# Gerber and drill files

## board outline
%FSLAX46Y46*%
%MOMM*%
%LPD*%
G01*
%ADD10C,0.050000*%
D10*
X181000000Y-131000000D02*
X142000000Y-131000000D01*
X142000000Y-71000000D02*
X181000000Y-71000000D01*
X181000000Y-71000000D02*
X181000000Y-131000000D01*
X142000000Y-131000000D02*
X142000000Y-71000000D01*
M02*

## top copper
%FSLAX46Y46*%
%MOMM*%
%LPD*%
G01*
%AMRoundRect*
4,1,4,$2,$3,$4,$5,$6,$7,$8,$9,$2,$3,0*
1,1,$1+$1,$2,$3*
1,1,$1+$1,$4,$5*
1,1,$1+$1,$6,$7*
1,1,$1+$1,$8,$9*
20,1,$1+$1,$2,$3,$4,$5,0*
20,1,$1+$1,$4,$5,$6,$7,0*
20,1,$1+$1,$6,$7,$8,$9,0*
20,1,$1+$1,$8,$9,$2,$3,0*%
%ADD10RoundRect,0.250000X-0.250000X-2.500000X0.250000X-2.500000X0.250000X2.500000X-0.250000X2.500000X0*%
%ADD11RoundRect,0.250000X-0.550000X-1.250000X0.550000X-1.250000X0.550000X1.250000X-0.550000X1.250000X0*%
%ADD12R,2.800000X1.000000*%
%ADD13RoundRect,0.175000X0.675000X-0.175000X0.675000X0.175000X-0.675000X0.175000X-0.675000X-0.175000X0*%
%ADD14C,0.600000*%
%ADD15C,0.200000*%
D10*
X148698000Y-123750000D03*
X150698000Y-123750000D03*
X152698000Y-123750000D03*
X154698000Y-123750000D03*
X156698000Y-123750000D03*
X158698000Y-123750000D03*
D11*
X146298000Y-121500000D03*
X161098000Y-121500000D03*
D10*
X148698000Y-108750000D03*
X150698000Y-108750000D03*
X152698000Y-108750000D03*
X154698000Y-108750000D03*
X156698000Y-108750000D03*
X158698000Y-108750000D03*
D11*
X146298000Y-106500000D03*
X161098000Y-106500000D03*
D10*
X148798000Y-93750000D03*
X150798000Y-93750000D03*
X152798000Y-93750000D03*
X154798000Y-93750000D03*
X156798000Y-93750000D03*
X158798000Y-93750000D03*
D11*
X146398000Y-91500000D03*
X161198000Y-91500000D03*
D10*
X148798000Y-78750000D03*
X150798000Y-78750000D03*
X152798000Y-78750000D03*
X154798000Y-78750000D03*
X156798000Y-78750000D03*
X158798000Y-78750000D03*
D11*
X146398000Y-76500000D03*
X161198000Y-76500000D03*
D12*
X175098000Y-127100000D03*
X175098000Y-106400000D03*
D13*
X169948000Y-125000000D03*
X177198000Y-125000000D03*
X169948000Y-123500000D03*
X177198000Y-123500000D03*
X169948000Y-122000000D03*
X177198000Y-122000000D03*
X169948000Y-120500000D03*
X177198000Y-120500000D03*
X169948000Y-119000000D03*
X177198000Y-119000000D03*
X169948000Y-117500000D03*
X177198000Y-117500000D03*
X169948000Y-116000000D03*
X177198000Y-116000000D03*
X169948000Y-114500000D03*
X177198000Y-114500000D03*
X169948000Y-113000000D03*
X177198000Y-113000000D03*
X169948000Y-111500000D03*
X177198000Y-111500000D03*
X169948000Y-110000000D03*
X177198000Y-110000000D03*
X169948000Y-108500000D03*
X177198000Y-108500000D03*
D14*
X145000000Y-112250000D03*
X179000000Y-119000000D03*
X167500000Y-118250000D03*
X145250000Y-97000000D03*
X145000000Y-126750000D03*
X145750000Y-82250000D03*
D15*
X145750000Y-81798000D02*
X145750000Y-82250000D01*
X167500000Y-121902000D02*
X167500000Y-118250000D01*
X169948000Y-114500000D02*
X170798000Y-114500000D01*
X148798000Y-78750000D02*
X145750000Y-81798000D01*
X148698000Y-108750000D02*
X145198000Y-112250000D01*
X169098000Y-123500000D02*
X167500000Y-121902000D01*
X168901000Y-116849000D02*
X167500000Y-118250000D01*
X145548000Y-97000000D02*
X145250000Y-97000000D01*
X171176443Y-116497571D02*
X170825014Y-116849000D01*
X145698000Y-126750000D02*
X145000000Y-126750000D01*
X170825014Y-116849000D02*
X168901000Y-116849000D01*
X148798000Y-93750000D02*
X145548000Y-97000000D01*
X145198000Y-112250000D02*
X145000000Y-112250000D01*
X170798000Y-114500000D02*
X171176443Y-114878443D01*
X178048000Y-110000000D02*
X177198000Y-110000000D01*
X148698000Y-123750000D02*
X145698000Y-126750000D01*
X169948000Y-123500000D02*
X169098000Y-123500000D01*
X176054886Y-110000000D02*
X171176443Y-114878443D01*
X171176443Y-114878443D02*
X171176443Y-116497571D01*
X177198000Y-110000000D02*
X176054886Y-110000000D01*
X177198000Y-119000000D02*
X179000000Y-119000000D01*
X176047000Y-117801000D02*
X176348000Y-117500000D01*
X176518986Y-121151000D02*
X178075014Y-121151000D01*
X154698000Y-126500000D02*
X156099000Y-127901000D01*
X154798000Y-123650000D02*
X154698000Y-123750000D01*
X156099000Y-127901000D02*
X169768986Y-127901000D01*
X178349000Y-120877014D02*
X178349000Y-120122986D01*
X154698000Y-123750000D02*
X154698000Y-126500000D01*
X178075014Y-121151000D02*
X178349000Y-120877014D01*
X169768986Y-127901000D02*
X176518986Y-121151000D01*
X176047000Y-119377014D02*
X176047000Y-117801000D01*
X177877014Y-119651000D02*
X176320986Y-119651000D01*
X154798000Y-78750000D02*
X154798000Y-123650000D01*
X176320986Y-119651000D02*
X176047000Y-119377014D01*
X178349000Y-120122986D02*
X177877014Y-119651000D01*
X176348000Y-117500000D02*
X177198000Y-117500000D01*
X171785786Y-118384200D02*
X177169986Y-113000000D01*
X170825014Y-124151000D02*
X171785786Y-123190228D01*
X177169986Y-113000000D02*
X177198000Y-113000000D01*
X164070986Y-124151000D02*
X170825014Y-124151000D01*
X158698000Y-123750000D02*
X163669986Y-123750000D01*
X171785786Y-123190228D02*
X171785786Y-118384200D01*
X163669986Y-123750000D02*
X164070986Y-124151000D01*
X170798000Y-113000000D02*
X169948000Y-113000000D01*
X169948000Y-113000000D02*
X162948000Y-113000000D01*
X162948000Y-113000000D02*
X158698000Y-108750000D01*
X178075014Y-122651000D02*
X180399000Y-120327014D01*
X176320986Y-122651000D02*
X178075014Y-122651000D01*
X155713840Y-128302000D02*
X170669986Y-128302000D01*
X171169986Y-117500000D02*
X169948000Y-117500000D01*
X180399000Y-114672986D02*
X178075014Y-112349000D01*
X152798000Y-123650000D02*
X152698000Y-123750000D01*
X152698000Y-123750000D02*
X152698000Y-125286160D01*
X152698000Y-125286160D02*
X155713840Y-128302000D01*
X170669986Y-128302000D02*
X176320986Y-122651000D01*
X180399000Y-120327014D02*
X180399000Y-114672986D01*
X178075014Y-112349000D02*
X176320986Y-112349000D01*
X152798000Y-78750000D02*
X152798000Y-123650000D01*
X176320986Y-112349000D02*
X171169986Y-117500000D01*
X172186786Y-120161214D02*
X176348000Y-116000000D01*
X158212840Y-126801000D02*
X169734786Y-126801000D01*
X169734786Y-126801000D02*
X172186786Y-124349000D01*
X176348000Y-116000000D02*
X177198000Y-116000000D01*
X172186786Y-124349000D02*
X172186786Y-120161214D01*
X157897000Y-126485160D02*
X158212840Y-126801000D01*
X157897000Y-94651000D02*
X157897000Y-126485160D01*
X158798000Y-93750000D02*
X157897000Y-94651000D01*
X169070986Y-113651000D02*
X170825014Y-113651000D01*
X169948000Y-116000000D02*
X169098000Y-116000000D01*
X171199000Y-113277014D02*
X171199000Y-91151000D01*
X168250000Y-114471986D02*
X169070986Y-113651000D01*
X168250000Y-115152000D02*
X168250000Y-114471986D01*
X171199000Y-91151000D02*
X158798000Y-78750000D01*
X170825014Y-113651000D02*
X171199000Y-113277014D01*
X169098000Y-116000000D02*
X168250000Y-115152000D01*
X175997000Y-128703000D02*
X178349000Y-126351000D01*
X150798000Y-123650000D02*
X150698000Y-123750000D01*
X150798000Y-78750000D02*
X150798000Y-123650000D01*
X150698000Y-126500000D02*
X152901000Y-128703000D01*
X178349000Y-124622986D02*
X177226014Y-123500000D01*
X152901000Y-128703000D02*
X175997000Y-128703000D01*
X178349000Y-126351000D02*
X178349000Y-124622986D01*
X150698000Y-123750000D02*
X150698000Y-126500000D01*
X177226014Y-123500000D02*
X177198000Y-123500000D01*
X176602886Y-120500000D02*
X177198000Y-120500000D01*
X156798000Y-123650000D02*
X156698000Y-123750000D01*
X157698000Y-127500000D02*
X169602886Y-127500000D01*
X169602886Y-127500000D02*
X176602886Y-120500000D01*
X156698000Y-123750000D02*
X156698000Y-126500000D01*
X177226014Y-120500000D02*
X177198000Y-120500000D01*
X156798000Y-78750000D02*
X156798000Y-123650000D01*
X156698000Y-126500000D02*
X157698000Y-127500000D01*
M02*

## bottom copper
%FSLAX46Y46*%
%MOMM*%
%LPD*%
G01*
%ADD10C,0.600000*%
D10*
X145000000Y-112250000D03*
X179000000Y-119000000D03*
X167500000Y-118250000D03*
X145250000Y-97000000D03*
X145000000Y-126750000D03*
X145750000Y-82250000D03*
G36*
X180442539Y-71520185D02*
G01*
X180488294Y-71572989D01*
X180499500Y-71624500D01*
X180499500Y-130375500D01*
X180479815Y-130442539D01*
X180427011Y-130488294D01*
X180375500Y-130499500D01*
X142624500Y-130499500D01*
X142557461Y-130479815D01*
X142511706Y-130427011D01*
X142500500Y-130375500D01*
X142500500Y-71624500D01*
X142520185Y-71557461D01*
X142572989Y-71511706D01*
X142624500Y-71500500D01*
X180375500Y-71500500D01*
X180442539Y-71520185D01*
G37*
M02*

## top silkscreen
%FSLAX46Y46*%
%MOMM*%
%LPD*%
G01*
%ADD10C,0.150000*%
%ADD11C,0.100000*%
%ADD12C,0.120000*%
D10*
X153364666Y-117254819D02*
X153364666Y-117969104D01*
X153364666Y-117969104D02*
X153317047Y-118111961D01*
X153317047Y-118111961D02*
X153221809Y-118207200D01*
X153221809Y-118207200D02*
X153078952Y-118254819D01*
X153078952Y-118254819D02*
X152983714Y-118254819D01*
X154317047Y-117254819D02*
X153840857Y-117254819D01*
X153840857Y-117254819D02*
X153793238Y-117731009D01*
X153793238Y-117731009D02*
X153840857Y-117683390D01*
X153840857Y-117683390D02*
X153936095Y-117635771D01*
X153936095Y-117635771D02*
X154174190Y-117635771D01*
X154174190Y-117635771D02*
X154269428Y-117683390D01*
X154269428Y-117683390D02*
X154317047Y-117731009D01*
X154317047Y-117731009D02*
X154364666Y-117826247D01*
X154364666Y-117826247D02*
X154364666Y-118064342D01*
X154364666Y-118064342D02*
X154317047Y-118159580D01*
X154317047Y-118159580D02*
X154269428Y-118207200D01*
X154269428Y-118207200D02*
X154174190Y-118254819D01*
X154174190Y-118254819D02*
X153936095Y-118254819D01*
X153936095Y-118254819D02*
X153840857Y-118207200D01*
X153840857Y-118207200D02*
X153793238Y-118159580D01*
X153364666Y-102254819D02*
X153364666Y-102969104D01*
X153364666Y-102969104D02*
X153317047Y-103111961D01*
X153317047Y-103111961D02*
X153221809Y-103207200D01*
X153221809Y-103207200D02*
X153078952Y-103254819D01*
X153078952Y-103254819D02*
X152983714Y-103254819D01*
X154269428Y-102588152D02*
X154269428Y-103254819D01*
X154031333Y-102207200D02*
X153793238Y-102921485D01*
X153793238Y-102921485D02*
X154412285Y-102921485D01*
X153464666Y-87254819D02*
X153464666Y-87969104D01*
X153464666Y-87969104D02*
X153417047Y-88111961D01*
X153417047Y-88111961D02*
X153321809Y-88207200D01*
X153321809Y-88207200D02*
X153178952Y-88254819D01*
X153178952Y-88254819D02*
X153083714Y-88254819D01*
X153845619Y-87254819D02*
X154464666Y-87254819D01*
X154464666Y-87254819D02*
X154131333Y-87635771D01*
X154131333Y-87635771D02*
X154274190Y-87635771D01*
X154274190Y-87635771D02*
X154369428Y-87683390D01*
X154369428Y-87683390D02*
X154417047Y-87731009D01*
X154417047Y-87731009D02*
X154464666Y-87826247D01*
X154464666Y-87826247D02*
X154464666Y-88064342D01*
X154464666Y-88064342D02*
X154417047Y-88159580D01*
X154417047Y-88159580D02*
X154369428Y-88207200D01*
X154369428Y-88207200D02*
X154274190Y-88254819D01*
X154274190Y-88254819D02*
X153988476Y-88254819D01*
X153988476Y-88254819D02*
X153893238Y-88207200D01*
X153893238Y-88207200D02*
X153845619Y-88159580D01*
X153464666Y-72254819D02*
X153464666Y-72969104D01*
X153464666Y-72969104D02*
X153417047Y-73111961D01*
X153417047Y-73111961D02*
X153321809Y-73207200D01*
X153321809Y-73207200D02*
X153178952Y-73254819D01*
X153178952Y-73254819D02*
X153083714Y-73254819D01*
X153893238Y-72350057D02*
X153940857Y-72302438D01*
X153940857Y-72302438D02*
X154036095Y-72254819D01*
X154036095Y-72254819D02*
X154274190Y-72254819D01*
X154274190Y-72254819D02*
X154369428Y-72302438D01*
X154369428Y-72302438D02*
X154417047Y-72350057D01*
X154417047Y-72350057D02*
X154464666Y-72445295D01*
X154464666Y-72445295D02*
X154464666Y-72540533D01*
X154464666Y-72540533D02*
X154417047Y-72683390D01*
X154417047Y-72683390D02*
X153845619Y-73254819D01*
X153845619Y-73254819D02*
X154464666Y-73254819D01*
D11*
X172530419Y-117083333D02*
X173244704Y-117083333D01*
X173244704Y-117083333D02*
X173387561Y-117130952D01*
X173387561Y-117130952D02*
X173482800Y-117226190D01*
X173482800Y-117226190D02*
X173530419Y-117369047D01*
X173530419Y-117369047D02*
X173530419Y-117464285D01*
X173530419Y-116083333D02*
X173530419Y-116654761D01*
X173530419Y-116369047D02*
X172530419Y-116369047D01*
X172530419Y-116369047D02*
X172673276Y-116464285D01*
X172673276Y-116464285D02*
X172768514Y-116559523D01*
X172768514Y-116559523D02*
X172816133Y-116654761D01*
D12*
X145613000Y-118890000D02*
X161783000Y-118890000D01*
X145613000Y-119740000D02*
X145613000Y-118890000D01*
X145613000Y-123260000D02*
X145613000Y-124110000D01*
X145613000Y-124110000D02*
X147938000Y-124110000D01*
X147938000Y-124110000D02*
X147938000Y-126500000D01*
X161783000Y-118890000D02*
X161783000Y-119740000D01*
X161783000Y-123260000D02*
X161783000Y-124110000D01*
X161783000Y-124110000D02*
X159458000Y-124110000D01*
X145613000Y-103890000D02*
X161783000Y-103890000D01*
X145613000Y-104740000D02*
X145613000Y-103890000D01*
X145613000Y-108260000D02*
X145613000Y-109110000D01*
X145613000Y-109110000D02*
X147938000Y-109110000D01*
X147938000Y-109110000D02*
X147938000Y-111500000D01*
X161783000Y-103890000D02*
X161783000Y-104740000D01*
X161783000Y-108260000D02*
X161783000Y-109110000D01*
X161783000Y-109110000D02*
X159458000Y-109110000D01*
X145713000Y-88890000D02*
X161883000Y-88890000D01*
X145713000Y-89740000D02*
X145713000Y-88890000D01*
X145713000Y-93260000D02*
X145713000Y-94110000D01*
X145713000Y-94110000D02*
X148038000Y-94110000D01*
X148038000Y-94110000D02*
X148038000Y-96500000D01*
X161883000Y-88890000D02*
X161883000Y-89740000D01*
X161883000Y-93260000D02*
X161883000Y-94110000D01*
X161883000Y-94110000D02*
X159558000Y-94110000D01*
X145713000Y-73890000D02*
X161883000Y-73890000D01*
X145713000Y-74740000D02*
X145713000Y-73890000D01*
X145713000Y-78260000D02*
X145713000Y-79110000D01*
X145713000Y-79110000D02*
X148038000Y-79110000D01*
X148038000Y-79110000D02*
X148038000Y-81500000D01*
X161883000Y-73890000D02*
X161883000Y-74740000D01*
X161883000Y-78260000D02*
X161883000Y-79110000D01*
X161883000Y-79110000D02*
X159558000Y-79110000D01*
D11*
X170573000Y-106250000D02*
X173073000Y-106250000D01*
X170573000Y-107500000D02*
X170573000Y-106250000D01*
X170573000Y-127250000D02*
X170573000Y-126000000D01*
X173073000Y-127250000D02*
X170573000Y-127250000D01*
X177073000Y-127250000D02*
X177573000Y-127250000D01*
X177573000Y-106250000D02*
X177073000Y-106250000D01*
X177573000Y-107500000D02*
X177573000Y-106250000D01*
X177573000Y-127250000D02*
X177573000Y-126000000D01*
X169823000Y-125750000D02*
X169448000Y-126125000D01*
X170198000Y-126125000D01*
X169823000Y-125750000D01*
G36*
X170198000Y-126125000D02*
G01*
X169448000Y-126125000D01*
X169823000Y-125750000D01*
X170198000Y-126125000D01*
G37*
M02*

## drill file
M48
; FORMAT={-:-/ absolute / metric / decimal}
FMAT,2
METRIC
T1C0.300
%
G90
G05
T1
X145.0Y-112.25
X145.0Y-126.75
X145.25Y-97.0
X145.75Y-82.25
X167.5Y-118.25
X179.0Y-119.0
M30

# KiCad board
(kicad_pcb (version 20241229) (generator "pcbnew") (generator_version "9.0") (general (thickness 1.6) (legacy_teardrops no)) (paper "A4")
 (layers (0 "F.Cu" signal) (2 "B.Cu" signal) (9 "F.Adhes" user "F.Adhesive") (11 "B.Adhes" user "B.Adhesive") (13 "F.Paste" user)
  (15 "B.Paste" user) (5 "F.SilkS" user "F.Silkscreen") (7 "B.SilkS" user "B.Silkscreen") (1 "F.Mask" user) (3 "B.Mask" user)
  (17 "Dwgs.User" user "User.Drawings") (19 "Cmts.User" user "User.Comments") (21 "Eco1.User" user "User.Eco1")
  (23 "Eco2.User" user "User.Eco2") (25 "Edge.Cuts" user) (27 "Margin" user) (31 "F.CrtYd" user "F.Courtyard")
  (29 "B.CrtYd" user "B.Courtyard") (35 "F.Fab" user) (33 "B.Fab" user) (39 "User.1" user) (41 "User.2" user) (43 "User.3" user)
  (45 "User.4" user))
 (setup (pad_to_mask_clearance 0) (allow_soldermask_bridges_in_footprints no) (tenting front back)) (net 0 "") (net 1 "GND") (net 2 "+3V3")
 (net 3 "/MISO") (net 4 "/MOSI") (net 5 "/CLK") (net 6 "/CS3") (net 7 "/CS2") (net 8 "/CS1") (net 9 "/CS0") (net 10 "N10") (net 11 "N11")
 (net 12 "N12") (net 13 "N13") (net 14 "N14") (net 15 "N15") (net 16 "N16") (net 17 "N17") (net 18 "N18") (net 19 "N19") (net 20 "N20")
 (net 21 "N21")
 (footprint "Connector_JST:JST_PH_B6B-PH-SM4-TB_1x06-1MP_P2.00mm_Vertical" (layer "F.Cu") (at 153.698 123.25)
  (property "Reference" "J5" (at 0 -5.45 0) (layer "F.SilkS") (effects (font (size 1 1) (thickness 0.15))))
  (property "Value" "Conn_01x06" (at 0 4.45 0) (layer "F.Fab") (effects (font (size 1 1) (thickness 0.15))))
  (fp_line (start -8.085 -4.36) (end 8.085 -4.36) (stroke (width 0.12) (type solid)) (layer "F.SilkS"))
  (fp_line (start -8.085 -3.51) (end -8.085 -4.36) (stroke (width 0.12) (type solid)) (layer "F.SilkS"))
  (fp_line (start -8.085 0.01) (end -8.085 0.86) (stroke (width 0.12) (type solid)) (layer "F.SilkS"))
  (fp_line (start -8.085 0.86) (end -5.76 0.86) (stroke (width 0.12) (type solid)) (layer "F.SilkS"))
  (fp_line (start -5.76 0.86) (end -5.76 3.25) (stroke (width 0.12) (type solid)) (layer "F.SilkS"))
  (fp_line (start 8.085 -4.36) (end 8.085 -3.51) (stroke (width 0.12) (type solid)) (layer "F.SilkS"))
  (fp_line (start 8.085 0.01) (end 8.085 0.86) (stroke (width 0.12) (type solid)) (layer "F.SilkS"))
  (fp_line (start 8.085 0.86) (end 5.76 0.86) (stroke (width 0.12) (type solid)) (layer "F.SilkS"))
  (pad "1" smd roundrect (at -5 0.5) (size 1 5.5) (layers "F.Cu" "F.Mask" "F.Paste") (roundrect_rratio 0.25) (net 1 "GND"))
  (pad "2" smd roundrect (at -3 0.5) (size 1 5.5) (layers "F.Cu" "F.Mask" "F.Paste") (roundrect_rratio 0.25) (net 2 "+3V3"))
  (pad "3" smd roundrect (at -1 0.5) (size 1 5.5) (layers "F.Cu" "F.Mask" "F.Paste") (roundrect_rratio 0.25) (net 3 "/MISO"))
  (pad "4" smd roundrect (at 1 0.5) (size 1 5.5) (layers "F.Cu" "F.Mask" "F.Paste") (roundrect_rratio 0.25) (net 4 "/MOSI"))
  (pad "5" smd roundrect (at 3 0.5) (size 1 5.5) (layers "F.Cu" "F.Mask" "F.Paste") (roundrect_rratio 0.25) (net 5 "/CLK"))
  (pad "6" smd roundrect (at 5 0.5) (size 1 5.5) (layers "F.Cu" "F.Mask" "F.Paste") (roundrect_rratio 0.25) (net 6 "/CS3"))
  (pad "MP" smd roundrect (at -7.4 -1.75) (size 1.6 3) (layers "F.Cu" "F.Mask" "F.Paste") (roundrect_rratio 0.15625))
  (pad "MP" smd roundrect (at 7.4 -1.75) (size 1.6 3) (layers "F.Cu" "F.Mask" "F.Paste") (roundrect_rratio 0.15625)))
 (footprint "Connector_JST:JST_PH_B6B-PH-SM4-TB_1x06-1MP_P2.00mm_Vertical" (layer "F.Cu") (at 153.698 108.25)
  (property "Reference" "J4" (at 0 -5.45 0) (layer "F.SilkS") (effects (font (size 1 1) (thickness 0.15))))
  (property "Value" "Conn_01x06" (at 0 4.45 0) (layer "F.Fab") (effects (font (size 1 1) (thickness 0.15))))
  (fp_line (start -8.085 -4.36) (end 8.085 -4.36) (stroke (width 0.12) (type solid)) (layer "F.SilkS"))
  (fp_line (start -8.085 -3.51) (end -8.085 -4.36) (stroke (width 0.12) (type solid)) (layer "F.SilkS"))
  (fp_line (start -8.085 0.01) (end -8.085 0.86) (stroke (width 0.12) (type solid)) (layer "F.SilkS"))
  (fp_line (start -8.085 0.86) (end -5.76 0.86) (stroke (width 0.12) (type solid)) (layer "F.SilkS"))
  (fp_line (start -5.76 0.86) (end -5.76 3.25) (stroke (width 0.12) (type solid)) (layer "F.SilkS"))
  (fp_line (start 8.085 -4.36) (end 8.085 -3.51) (stroke (width 0.12) (type solid)) (layer "F.SilkS"))
  (fp_line (start 8.085 0.01) (end 8.085 0.86) (stroke (width 0.12) (type solid)) (layer "F.SilkS"))
  (fp_line (start 8.085 0.86) (end 5.76 0.86) (stroke (width 0.12) (type solid)) (layer "F.SilkS"))
  (pad "1" smd roundrect (at -5 0.5) (size 1 5.5) (layers "F.Cu" "F.Mask" "F.Paste") (roundrect_rratio 0.25) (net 1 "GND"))
  (pad "2" smd roundrect (at -3 0.5) (size 1 5.5) (layers "F.Cu" "F.Mask" "F.Paste") (roundrect_rratio 0.25) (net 2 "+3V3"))
  (pad "3" smd roundrect (at -1 0.5) (size 1 5.5) (layers "F.Cu" "F.Mask" "F.Paste") (roundrect_rratio 0.25) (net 3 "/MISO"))
  (pad "4" smd roundrect (at 1 0.5) (size 1 5.5) (layers "F.Cu" "F.Mask" "F.Paste") (roundrect_rratio 0.25) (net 4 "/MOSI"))
  (pad "5" smd roundrect (at 3 0.5) (size 1 5.5) (layers "F.Cu" "F.Mask" "F.Paste") (roundrect_rratio 0.25) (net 5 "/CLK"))
  (pad "6" smd roundrect (at 5 0.5) (size 1 5.5) (layers "F.Cu" "F.Mask" "F.Paste") (roundrect_rratio 0.25) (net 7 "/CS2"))
  (pad "MP" smd roundrect (at -7.4 -1.75) (size 1.6 3) (layers "F.Cu" "F.Mask" "F.Paste") (roundrect_rratio 0.15625))
  (pad "MP" smd roundrect (at 7.4 -1.75) (size 1.6 3) (layers "F.Cu" "F.Mask" "F.Paste") (roundrect_rratio 0.15625)))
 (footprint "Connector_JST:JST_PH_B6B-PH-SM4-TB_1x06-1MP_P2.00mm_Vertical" (layer "F.Cu") (at 153.798 93.25)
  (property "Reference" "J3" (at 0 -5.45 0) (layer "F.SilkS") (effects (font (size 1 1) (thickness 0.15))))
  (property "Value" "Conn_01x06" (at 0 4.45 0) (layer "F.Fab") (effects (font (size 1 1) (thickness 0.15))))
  (fp_line (start -8.085 -4.36) (end 8.085 -4.36) (stroke (width 0.12) (type solid)) (layer "F.SilkS"))
  (fp_line (start -8.085 -3.51) (end -8.085 -4.36) (stroke (width 0.12) (type solid)) (layer "F.SilkS"))
  (fp_line (start -8.085 0.01) (end -8.085 0.86) (stroke (width 0.12) (type solid)) (layer "F.SilkS"))
  (fp_line (start -8.085 0.86) (end -5.76 0.86) (stroke (width 0.12) (type solid)) (layer "F.SilkS"))
  (fp_line (start -5.76 0.86) (end -5.76 3.25) (stroke (width 0.12) (type solid)) (layer "F.SilkS"))
  (fp_line (start 8.085 -4.36) (end 8.085 -3.51) (stroke (width 0.12) (type solid)) (layer "F.SilkS"))
  (fp_line (start 8.085 0.01) (end 8.085 0.86) (stroke (width 0.12) (type solid)) (layer "F.SilkS"))
  (fp_line (start 8.085 0.86) (end 5.76 0.86) (stroke (width 0.12) (type solid)) (layer "F.SilkS"))
  (pad "1" smd roundrect (at -5 0.5) (size 1 5.5) (layers "F.Cu" "F.Mask" "F.Paste") (roundrect_rratio 0.25) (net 1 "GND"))
  (pad "2" smd roundrect (at -3 0.5) (size 1 5.5) (layers "F.Cu" "F.Mask" "F.Paste") (roundrect_rratio 0.25) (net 2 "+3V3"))
  (pad "3" smd roundrect (at -1 0.5) (size 1 5.5) (layers "F.Cu" "F.Mask" "F.Paste") (roundrect_rratio 0.25) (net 3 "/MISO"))
  (pad "4" smd roundrect (at 1 0.5) (size 1 5.5) (layers "F.Cu" "F.Mask" "F.Paste") (roundrect_rratio 0.25) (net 4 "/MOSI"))
  (pad "5" smd roundrect (at 3 0.5) (size 1 5.5) (layers "F.Cu" "F.Mask" "F.Paste") (roundrect_rratio 0.25) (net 5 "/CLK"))
  (pad "6" smd roundrect (at 5 0.5) (size 1 5.5) (layers "F.Cu" "F.Mask" "F.Paste") (roundrect_rratio 0.25) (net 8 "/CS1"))
  (pad "MP" smd roundrect (at -7.4 -1.75) (size 1.6 3) (layers "F.Cu" "F.Mask" "F.Paste") (roundrect_rratio 0.15625))
  (pad "MP" smd roundrect (at 7.4 -1.75) (size 1.6 3) (layers "F.Cu" "F.Mask" "F.Paste") (roundrect_rratio 0.15625)))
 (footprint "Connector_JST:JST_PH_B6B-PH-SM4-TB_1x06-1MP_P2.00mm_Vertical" (layer "F.Cu") (at 153.798 78.25)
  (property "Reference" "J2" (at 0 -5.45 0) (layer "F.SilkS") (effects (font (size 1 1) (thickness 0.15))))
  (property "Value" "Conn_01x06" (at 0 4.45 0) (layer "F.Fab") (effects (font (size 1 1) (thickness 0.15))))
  (fp_line (start -8.085 -4.36) (end 8.085 -4.36) (stroke (width 0.12) (type solid)) (layer "F.SilkS"))
  (fp_line (start -8.085 -3.51) (end -8.085 -4.36) (stroke (width 0.12) (type solid)) (layer "F.SilkS"))
  (fp_line (start -8.085 0.01) (end -8.085 0.86) (stroke (width 0.12) (type solid)) (layer "F.SilkS"))
  (fp_line (start -8.085 0.86) (end -5.76 0.86) (stroke (width 0.12) (type solid)) (layer "F.SilkS"))
  (fp_line (start -5.76 0.86) (end -5.76 3.25) (stroke (width 0.12) (type solid)) (layer "F.SilkS"))
  (fp_line (start 8.085 -4.36) (end 8.085 -3.51) (stroke (width 0.12) (type solid)) (layer "F.SilkS"))
  (fp_line (start 8.085 0.01) (end 8.085 0.86) (stroke (width 0.12) (type solid)) (layer "F.SilkS"))
  (fp_line (start 8.085 0.86) (end 5.76 0.86) (stroke (width 0.12) (type solid)) (layer "F.SilkS"))
  (pad "1" smd roundrect (at -5 0.5) (size 1 5.5) (layers "F.Cu" "F.Mask" "F.Paste") (roundrect_rratio 0.25) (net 1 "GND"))
  (pad "2" smd roundrect (at -3 0.5) (size 1 5.5) (layers "F.Cu" "F.Mask" "F.Paste") (roundrect_rratio 0.25) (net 2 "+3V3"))
  (pad "3" smd roundrect (at -1 0.5) (size 1 5.5) (layers "F.Cu" "F.Mask" "F.Paste") (roundrect_rratio 0.25) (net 3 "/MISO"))
  (pad "4" smd roundrect (at 1 0.5) (size 1 5.5) (layers "F.Cu" "F.Mask" "F.Paste") (roundrect_rratio 0.25) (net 4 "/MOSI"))
  (pad "5" smd roundrect (at 3 0.5) (size 1 5.5) (layers "F.Cu" "F.Mask" "F.Paste") (roundrect_rratio 0.25) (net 5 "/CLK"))
  (pad "6" smd roundrect (at 5 0.5) (size 1 5.5) (layers "F.Cu" "F.Mask" "F.Paste") (roundrect_rratio 0.25) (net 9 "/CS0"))
  (pad "MP" smd roundrect (at -7.4 -1.75) (size 1.6 3) (layers "F.Cu" "F.Mask" "F.Paste") (roundrect_rratio 0.15625))
  (pad "MP" smd roundrect (at 7.4 -1.75) (size 1.6 3) (layers "F.Cu" "F.Mask" "F.Paste") (roundrect_rratio 0.15625)))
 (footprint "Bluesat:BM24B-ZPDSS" (layer "F.Cu") (at 173.573 116.75 90)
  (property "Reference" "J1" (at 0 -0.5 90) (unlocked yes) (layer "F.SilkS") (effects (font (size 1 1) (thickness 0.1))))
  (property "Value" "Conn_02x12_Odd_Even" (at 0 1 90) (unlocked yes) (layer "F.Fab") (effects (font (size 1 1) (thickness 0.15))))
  (fp_line (start 10.5 -3) (end 10.5 -0.5) (stroke (width 0.1) (type default)) (layer "F.SilkS"))
  (fp_line (start 9.25 -3) (end 10.5 -3) (stroke (width 0.1) (type default)) (layer "F.SilkS"))
  (fp_line (start -10.5 -3) (end -9.25 -3) (stroke (width 0.1) (type default)) (layer "F.SilkS"))
  (fp_line (start -10.5 -0.5) (end -10.5 -3) (stroke (width 0.1) (type default)) (layer "F.SilkS"))
  (fp_line (start -10.5 3.5) (end -10.5 4) (stroke (width 0.1) (type default)) (layer "F.SilkS"))
  (fp_line (start 10.5 4) (end 10.5 3.5) (stroke (width 0.1) (type default)) (layer "F.SilkS"))
  (fp_line (start 9.25 4) (end 10.5 4) (stroke (width 0.1) (type default)) (layer "F.SilkS"))
  (fp_line (start -10.5 4) (end -9.25 4) (stroke (width 0.1) (type default)) (layer "F.SilkS"))
  (fp_poly (pts (xy -9 -3.75) (xy -9.375 -4.125) (xy -9.375 -3.375)) (stroke (width 0.1) (type solid)) (fill yes) (layer "F.SilkS"))
  (pad "" smd rect (at -10.35 1.525 90) (size 1 2.8) (layers "F.Cu" "F.Mask" "F.Paste") (thermal_bridge_angle 45))
  (pad "" smd rect (at 10.35 1.525 90) (size 1 2.8) (layers "F.Cu" "F.Mask" "F.Paste") (thermal_bridge_angle 45))
  (pad "1" smd roundrect (at -8.25 -3.625 90) (size 0.7 1.7) (layers "F.Cu" "F.Mask" "F.Paste") (roundrect_rratio 0.25) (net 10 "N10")
   (thermal_bridge_angle 45))
  (pad "2" smd roundrect (at -8.25 3.625 90) (size 0.7 1.7) (layers "F.Cu" "F.Mask" "F.Paste") (roundrect_rratio 0.25) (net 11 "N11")
   (thermal_bridge_angle 45))
  (pad "3" smd roundrect (at -6.75 -3.625 90) (size 0.7 1.7) (layers "F.Cu" "F.Mask" "F.Paste") (roundrect_rratio 0.25) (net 1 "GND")
   (thermal_bridge_angle 45))
  (pad "4" smd roundrect (at -6.75 3.625 90) (size 0.7 1.7) (layers "F.Cu" "F.Mask" "F.Paste") (roundrect_rratio 0.25) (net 2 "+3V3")
   (thermal_bridge_angle 45))
  (pad "5" smd roundrect (at -5.25 -3.625 90) (size 0.7 1.7) (layers "F.Cu" "F.Mask" "F.Paste") (roundrect_rratio 0.25) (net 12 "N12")
   (thermal_bridge_angle 45))
  (pad "6" smd roundrect (at -5.25 3.625 90) (size 0.7 1.7) (layers "F.Cu" "F.Mask" "F.Paste") (roundrect_rratio 0.25) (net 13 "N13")
   (thermal_bridge_angle 45))
  (pad "7" smd roundrect (at -3.75 -3.625 90) (size 0.7 1.7) (layers "F.Cu" "F.Mask" "F.Paste") (roundrect_rratio 0.25) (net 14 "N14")
   (thermal_bridge_angle 45))
  (pad "8" smd roundrect (at -3.75 3.625 90) (size 0.7 1.7) (layers "F.Cu" "F.Mask" "F.Paste") (roundrect_rratio 0.25) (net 5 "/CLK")
   (thermal_bridge_angle 45))
  (pad "9" smd roundrect (at -2.25 -3.625 90) (size 0.7 1.7) (layers "F.Cu" "F.Mask" "F.Paste") (roundrect_rratio 0.25) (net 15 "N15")
   (thermal_bridge_angle 45))
  (pad "10" smd roundrect (at -2.25 3.625 90) (size 0.7 1.7) (layers "F.Cu" "F.Mask" "F.Paste") (roundrect_rratio 0.25) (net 1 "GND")
   (thermal_bridge_angle 45))
  (pad "11" smd roundrect (at -0.75 -3.625 90) (size 0.7 1.7) (layers "F.Cu" "F.Mask" "F.Paste") (roundrect_rratio 0.25) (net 3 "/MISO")
   (thermal_bridge_angle 45))
  (pad "12" smd roundrect (at -0.75 3.625 90) (size 0.7 1.7) (layers "F.Cu" "F.Mask" "F.Paste") (roundrect_rratio 0.25) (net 4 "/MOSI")
   (thermal_bridge_angle 45))
  (pad "13" smd roundrect (at 0.75 -3.625 90) (size 0.7 1.7) (layers "F.Cu" "F.Mask" "F.Paste") (roundrect_rratio 0.25) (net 9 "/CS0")
   (thermal_bridge_angle 45))
  (pad "14" smd roundrect (at 0.75 3.625 90) (size 0.7 1.7) (layers "F.Cu" "F.Mask" "F.Paste") (roundrect_rratio 0.25) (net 8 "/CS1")
   (thermal_bridge_angle 45))
  (pad "15" smd roundrect (at 2.25 -3.625 90) (size 0.7 1.7) (layers "F.Cu" "F.Mask" "F.Paste") (roundrect_rratio 0.25) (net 1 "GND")
   (thermal_bridge_angle 45))
  (pad "16" smd roundrect (at 2.25 3.625 90) (size 0.7 1.7) (layers "F.Cu" "F.Mask" "F.Paste") (roundrect_rratio 0.25) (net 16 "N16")
   (thermal_bridge_angle 45))
  (pad "17" smd roundrect (at 3.75 -3.625 90) (size 0.7 1.7) (layers "F.Cu" "F.Mask" "F.Paste") (roundrect_rratio 0.25) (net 7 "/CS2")
   (thermal_bridge_angle 45))
  (pad "18" smd roundrect (at 3.75 3.625 90) (size 0.7 1.7) (layers "F.Cu" "F.Mask" "F.Paste") (roundrect_rratio 0.25) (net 6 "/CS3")
   (thermal_bridge_angle 45))
  (pad "19" smd roundrect (at 5.25 -3.625 90) (size 0.7 1.7) (layers "F.Cu" "F.Mask" "F.Paste") (roundrect_rratio 0.25) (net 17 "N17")
   (thermal_bridge_angle 45))
  (pad "20" smd roundrect (at 5.25 3.625 90) (size 0.7 1.7) (layers "F.Cu" "F.Mask" "F.Paste") (roundrect_rratio 0.25) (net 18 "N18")
   (thermal_bridge_angle 45))
  (pad "21" smd roundrect (at 6.75 -3.625 90) (size 0.7 1.7) (layers "F.Cu" "F.Mask" "F.Paste") (roundrect_rratio 0.25) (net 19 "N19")
   (thermal_bridge_angle 45))
  (pad "22" smd roundrect (at 6.75 3.625 90) (size 0.7 1.7) (layers "F.Cu" "F.Mask" "F.Paste") (roundrect_rratio 0.25) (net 1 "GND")
   (thermal_bridge_angle 45))
  (pad "23" smd roundrect (at 8.25 -3.625 90) (size 0.7 1.7) (layers "F.Cu" "F.Mask" "F.Paste") (roundrect_rratio 0.25) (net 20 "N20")
   (thermal_bridge_angle 45))
  (pad "24" smd roundrect (at 8.25 3.625 90) (size 0.7 1.7) (layers "F.Cu" "F.Mask" "F.Paste") (roundrect_rratio 0.25) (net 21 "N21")
   (thermal_bridge_angle 45)))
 (gr_line (start 181 131) (end 142 131) (stroke (width 0.05) (type default)) (layer "Edge.Cuts"))
 (gr_line (start 142 71) (end 181 71) (stroke (width 0.05) (type default)) (layer "Edge.Cuts"))
 (gr_line (start 181 71) (end 181 131) (stroke (width 0.05) (type solid)) (layer "Edge.Cuts"))
 (gr_line (start 142 131) (end 142 71) (stroke (width 0.05) (type default)) (layer "Edge.Cuts"))
 (segment (start 145.75 81.798) (end 145.75 82.25) (width 0.2) (layer "F.Cu") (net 1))
 (segment (start 167.5 121.902) (end 167.5 118.25) (width 0.2) (layer "F.Cu") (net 1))
 (segment (start 169.948 114.5) (end 170.798 114.5) (width 0.2) (layer "F.Cu") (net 1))
 (segment (start 148.798 78.75) (end 145.75 81.798) (width 0.2) (layer "F.Cu") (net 1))
 (segment (start 148.698 108.75) (end 145.198 112.25) (width 0.2) (layer "F.Cu") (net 1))
 (segment (start 169.098 123.5) (end 167.5 121.902) (width 0.2) (layer "F.Cu") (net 1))
 (segment (start 168.901 116.849) (end 167.5 118.25) (width 0.2) (layer "F.Cu") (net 1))
 (segment (start 145.548 97) (end 145.25 97) (width 0.2) (layer "F.Cu") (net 1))
 (segment (start 171.176443 116.497571) (end 170.825014 116.849) (width 0.2) (layer "F.Cu") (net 1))
 (segment (start 145.698 126.75) (end 145 126.75) (width 0.2) (layer "F.Cu") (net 1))
 (segment (start 170.825014 116.849) (end 168.901 116.849) (width 0.2) (layer "F.Cu") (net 1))
 (segment (start 148.798 93.75) (end 145.548 97) (width 0.2) (layer "F.Cu") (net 1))
 (segment (start 145.198 112.25) (end 145 112.25) (width 0.2) (layer "F.Cu") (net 1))
 (segment (start 170.798 114.5) (end 171.176443 114.878443) (width 0.2) (layer "F.Cu") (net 1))
 (segment (start 178.048 110) (end 177.198 110) (width 0.2) (layer "F.Cu") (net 1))
 (segment (start 148.698 123.75) (end 145.698 126.75) (width 0.2) (layer "F.Cu") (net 1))
 (segment (start 169.948 123.5) (end 169.098 123.5) (width 0.2) (layer "F.Cu") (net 1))
 (segment (start 176.054886 110) (end 171.176443 114.878443) (width 0.2) (layer "F.Cu") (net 1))
 (segment (start 171.176443 114.878443) (end 171.176443 116.497571) (width 0.2) (layer "F.Cu") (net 1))
 (segment (start 177.198 110) (end 176.054886 110) (width 0.2) (layer "F.Cu") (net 1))
 (segment (start 177.198 119) (end 179 119) (width 0.2) (layer "F.Cu") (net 1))
 (via (at 145 112.25) (size 0.6) (drill 0.3) (layers "F.Cu" "B.Cu") (free yes) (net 1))
 (via (at 179 119) (size 0.6) (drill 0.3) (layers "F.Cu" "B.Cu") (free yes) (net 1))
 (via (at 167.5 118.25) (size 0.6) (drill 0.3) (layers "F.Cu" "B.Cu") (free yes) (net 1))
 (via (at 145.25 97) (size 0.6) (drill 0.3) (layers "F.Cu" "B.Cu") (free yes) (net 1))
 (via (at 145 126.75) (size 0.6) (drill 0.3) (layers "F.Cu" "B.Cu") (free yes) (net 1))
 (via (at 145.75 82.25) (size 0.6) (drill 0.3) (layers "F.Cu" "B.Cu") (free yes) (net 1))
 (segment (start 176.047 117.801) (end 176.348 117.5) (width 0.2) (layer "F.Cu") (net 4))
 (segment (start 176.518986 121.151) (end 178.075014 121.151) (width 0.2) (layer "F.Cu") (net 4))
 (segment (start 154.698 126.5) (end 156.099 127.901) (width 0.2) (layer "F.Cu") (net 4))
 (segment (start 154.798 123.65) (end 154.698 123.75) (width 0.2) (layer "F.Cu") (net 4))
 (segment (start 156.099 127.901) (end 169.768986 127.901) (width 0.2) (layer "F.Cu") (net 4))
 (segment (start 178.349 120.877014) (end 178.349 120.122986) (width 0.2) (layer "F.Cu") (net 4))
 (segment (start 154.698 123.75) (end 154.698 126.5) (width 0.2) (layer "F.Cu") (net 4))
 (segment (start 178.075014 121.151) (end 178.349 120.877014) (width 0.2) (layer "F.Cu") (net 4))
 (segment (start 169.768986 127.901) (end 176.518986 121.151) (width 0.2) (layer "F.Cu") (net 4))
 (segment (start 176.047 119.377014) (end 176.047 117.801) (width 0.2) (layer "F.Cu") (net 4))
 (segment (start 177.877014 119.651) (end 176.320986 119.651) (width 0.2) (layer "F.Cu") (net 4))
 (segment (start 154.798 78.75) (end 154.798 123.65) (width 0.2) (layer "F.Cu") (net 4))
 (segment (start 176.320986 119.651) (end 176.047 119.377014) (width 0.2) (layer "F.Cu") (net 4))
 (segment (start 178.349 120.122986) (end 177.877014 119.651) (width 0.2) (layer "F.Cu") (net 4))
 (segment (start 176.348 117.5) (end 177.198 117.5) (width 0.2) (layer "F.Cu") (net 4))
 (segment (start 171.785786 118.3842) (end 177.169986 113) (width 0.2) (layer "F.Cu") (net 6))
 (segment (start 170.825014 124.151) (end 171.785786 123.190228) (width 0.2) (layer "F.Cu") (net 6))
 (segment (start 177.169986 113) (end 177.198 113) (width 0.2) (layer "F.Cu") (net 6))
 (segment (start 164.070986 124.151) (end 170.825014 124.151) (width 0.2) (layer "F.Cu") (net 6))
 (segment (start 158.698 123.75) (end 163.669986 123.75) (width 0.2) (layer "F.Cu") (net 6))
 (segment (start 171.785786 123.190228) (end 171.785786 118.3842) (width 0.2) (layer "F.Cu") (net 6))
 (segment (start 163.669986 123.75) (end 164.070986 124.151) (width 0.2) (layer "F.Cu") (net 6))
 (segment (start 170.798 113) (end 169.948 113) (width 0.2) (layer "F.Cu") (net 7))
 (segment (start 169.948 113) (end 162.948 113) (width 0.2) (layer "F.Cu") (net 7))
 (segment (start 162.948 113) (end 158.698 108.75) (width 0.2) (layer "F.Cu") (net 7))
 (segment (start 178.075014 122.651) (end 180.399 120.327014) (width 0.2) (layer "F.Cu") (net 3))
 (segment (start 176.320986 122.651) (end 178.075014 122.651) (width 0.2) (layer "F.Cu") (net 3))
 (segment (start 155.71384 128.302) (end 170.669986 128.302) (width 0.2) (layer "F.Cu") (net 3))
 (segment (start 171.169986 117.5) (end 169.948 117.5) (width 0.2) (layer "F.Cu") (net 3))
 (segment (start 180.399 114.672986) (end 178.075014 112.349) (width 0.2) (layer "F.Cu") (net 3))
 (segment (start 152.798 123.65) (end 152.698 123.75) (width 0.2) (layer "F.Cu") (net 3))
 (segment (start 152.698 123.75) (end 152.698 125.28616) (width 0.2) (layer "F.Cu") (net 3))
 (segment (start 152.698 125.28616) (end 155.71384 128.302) (width 0.2) (layer "F.Cu") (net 3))
 (segment (start 170.669986 128.302) (end 176.320986 122.651) (width 0.2) (layer "F.Cu") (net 3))
 (segment (start 180.399 120.327014) (end 180.399 114.672986) (width 0.2) (layer "F.Cu") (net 3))
 (segment (start 178.075014 112.349) (end 176.320986 112.349) (width 0.2) (layer "F.Cu") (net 3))
 (segment (start 152.798 78.75) (end 152.798 123.65) (width 0.2) (layer "F.Cu") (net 3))
 (segment (start 176.320986 112.349) (end 171.169986 117.5) (width 0.2) (layer "F.Cu") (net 3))
 (segment (start 172.186786 120.161214) (end 176.348 116) (width 0.2) (layer "F.Cu") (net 8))
 (segment (start 158.21284 126.801) (end 169.734786 126.801) (width 0.2) (layer "F.Cu") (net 8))
 (segment (start 169.734786 126.801) (end 172.186786 124.349) (width 0.2) (layer "F.Cu") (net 8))
 (segment (start 176.348 116) (end 177.198 116) (width 0.2) (layer "F.Cu") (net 8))
 (segment (start 172.186786 124.349) (end 172.186786 120.161214) (width 0.2) (layer "F.Cu") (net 8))
 (segment (start 157.897 126.48516) (end 158.21284 126.801) (width 0.2) (layer "F.Cu") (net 8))
 (segment (start 157.897 94.651) (end 157.897 126.48516) (width 0.2) (layer "F.Cu") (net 8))
 (segment (start 158.798 93.75) (end 157.897 94.651) (width 0.2) (layer "F.Cu") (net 8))
 (segment (start 169.070986 113.651) (end 170.825014 113.651) (width 0.2) (layer "F.Cu") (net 9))
 (segment (start 169.948 116) (end 169.098 116) (width 0.2) (layer "F.Cu") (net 9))
 (segment (start 171.199 113.277014) (end 171.199 91.151) (width 0.2) (layer "F.Cu") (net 9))
 (segment (start 168.25 114.471986) (end 169.070986 113.651) (width 0.2) (layer "F.Cu") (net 9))
 (segment (start 168.25 115.152) (end 168.25 114.471986) (width 0.2) (layer "F.Cu") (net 9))
 (segment (start 171.199 91.151) (end 158.798 78.75) (width 0.2) (layer "F.Cu") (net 9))
 (segment (start 170.825014 113.651) (end 171.199 113.277014) (width 0.2) (layer "F.Cu") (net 9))
 (segment (start 169.098 116) (end 168.25 115.152) (width 0.2) (layer "F.Cu") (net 9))
 (segment (start 175.997 128.703) (end 178.349 126.351) (width 0.2) (layer "F.Cu") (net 2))
 (segment (start 150.798 123.65) (end 150.698 123.75) (width 0.2) (layer "F.Cu") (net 2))
 (segment (start 150.798 78.75) (end 150.798 123.65) (width 0.2) (layer "F.Cu") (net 2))
 (segment (start 150.698 126.5) (end 152.901 128.703) (width 0.2) (layer "F.Cu") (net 2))
 (segment (start 178.349 124.622986) (end 177.226014 123.5) (width 0.2) (layer "F.Cu") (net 2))
 (segment (start 152.901 128.703) (end 175.997 128.703) (width 0.2) (layer "F.Cu") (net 2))
 (segment (start 178.349 126.351) (end 178.349 124.622986) (width 0.2) (layer "F.Cu") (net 2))
 (segment (start 150.698 123.75) (end 150.698 126.5) (width 0.2) (layer "F.Cu") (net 2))
 (segment (start 177.226014 123.5) (end 177.198 123.5) (width 0.2) (layer "F.Cu") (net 2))
 (segment (start 176.602886 120.5) (end 177.198 120.5) (width 0.2) (layer "F.Cu") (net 5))
 (segment (start 156.798 123.65) (end 156.698 123.75) (width 0.2) (layer "F.Cu") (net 5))
 (segment (start 157.698 127.5) (end 169.602886 127.5) (width 0.2) (layer "F.Cu") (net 5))
 (segment (start 169.602886 127.5) (end 176.602886 120.5) (width 0.2) (layer "F.Cu") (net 5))
 (segment (start 156.698 123.75) (end 156.698 126.5) (width 0.2) (layer "F.Cu") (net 5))
 (segment (start 177.226014 120.5) (end 177.198 120.5) (width 0.2) (layer "F.Cu") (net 5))
 (segment (start 156.798 78.75) (end 156.798 123.65) (width 0.2) (layer "F.Cu") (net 5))
 (segment (start 156.698 126.5) (end 157.698 127.5) (width 0.2) (layer "F.Cu") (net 5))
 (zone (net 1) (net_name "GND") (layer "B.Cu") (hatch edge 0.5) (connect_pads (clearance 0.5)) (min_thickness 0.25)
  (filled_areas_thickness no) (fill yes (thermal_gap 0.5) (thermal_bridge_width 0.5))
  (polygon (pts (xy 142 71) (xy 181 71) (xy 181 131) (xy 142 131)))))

